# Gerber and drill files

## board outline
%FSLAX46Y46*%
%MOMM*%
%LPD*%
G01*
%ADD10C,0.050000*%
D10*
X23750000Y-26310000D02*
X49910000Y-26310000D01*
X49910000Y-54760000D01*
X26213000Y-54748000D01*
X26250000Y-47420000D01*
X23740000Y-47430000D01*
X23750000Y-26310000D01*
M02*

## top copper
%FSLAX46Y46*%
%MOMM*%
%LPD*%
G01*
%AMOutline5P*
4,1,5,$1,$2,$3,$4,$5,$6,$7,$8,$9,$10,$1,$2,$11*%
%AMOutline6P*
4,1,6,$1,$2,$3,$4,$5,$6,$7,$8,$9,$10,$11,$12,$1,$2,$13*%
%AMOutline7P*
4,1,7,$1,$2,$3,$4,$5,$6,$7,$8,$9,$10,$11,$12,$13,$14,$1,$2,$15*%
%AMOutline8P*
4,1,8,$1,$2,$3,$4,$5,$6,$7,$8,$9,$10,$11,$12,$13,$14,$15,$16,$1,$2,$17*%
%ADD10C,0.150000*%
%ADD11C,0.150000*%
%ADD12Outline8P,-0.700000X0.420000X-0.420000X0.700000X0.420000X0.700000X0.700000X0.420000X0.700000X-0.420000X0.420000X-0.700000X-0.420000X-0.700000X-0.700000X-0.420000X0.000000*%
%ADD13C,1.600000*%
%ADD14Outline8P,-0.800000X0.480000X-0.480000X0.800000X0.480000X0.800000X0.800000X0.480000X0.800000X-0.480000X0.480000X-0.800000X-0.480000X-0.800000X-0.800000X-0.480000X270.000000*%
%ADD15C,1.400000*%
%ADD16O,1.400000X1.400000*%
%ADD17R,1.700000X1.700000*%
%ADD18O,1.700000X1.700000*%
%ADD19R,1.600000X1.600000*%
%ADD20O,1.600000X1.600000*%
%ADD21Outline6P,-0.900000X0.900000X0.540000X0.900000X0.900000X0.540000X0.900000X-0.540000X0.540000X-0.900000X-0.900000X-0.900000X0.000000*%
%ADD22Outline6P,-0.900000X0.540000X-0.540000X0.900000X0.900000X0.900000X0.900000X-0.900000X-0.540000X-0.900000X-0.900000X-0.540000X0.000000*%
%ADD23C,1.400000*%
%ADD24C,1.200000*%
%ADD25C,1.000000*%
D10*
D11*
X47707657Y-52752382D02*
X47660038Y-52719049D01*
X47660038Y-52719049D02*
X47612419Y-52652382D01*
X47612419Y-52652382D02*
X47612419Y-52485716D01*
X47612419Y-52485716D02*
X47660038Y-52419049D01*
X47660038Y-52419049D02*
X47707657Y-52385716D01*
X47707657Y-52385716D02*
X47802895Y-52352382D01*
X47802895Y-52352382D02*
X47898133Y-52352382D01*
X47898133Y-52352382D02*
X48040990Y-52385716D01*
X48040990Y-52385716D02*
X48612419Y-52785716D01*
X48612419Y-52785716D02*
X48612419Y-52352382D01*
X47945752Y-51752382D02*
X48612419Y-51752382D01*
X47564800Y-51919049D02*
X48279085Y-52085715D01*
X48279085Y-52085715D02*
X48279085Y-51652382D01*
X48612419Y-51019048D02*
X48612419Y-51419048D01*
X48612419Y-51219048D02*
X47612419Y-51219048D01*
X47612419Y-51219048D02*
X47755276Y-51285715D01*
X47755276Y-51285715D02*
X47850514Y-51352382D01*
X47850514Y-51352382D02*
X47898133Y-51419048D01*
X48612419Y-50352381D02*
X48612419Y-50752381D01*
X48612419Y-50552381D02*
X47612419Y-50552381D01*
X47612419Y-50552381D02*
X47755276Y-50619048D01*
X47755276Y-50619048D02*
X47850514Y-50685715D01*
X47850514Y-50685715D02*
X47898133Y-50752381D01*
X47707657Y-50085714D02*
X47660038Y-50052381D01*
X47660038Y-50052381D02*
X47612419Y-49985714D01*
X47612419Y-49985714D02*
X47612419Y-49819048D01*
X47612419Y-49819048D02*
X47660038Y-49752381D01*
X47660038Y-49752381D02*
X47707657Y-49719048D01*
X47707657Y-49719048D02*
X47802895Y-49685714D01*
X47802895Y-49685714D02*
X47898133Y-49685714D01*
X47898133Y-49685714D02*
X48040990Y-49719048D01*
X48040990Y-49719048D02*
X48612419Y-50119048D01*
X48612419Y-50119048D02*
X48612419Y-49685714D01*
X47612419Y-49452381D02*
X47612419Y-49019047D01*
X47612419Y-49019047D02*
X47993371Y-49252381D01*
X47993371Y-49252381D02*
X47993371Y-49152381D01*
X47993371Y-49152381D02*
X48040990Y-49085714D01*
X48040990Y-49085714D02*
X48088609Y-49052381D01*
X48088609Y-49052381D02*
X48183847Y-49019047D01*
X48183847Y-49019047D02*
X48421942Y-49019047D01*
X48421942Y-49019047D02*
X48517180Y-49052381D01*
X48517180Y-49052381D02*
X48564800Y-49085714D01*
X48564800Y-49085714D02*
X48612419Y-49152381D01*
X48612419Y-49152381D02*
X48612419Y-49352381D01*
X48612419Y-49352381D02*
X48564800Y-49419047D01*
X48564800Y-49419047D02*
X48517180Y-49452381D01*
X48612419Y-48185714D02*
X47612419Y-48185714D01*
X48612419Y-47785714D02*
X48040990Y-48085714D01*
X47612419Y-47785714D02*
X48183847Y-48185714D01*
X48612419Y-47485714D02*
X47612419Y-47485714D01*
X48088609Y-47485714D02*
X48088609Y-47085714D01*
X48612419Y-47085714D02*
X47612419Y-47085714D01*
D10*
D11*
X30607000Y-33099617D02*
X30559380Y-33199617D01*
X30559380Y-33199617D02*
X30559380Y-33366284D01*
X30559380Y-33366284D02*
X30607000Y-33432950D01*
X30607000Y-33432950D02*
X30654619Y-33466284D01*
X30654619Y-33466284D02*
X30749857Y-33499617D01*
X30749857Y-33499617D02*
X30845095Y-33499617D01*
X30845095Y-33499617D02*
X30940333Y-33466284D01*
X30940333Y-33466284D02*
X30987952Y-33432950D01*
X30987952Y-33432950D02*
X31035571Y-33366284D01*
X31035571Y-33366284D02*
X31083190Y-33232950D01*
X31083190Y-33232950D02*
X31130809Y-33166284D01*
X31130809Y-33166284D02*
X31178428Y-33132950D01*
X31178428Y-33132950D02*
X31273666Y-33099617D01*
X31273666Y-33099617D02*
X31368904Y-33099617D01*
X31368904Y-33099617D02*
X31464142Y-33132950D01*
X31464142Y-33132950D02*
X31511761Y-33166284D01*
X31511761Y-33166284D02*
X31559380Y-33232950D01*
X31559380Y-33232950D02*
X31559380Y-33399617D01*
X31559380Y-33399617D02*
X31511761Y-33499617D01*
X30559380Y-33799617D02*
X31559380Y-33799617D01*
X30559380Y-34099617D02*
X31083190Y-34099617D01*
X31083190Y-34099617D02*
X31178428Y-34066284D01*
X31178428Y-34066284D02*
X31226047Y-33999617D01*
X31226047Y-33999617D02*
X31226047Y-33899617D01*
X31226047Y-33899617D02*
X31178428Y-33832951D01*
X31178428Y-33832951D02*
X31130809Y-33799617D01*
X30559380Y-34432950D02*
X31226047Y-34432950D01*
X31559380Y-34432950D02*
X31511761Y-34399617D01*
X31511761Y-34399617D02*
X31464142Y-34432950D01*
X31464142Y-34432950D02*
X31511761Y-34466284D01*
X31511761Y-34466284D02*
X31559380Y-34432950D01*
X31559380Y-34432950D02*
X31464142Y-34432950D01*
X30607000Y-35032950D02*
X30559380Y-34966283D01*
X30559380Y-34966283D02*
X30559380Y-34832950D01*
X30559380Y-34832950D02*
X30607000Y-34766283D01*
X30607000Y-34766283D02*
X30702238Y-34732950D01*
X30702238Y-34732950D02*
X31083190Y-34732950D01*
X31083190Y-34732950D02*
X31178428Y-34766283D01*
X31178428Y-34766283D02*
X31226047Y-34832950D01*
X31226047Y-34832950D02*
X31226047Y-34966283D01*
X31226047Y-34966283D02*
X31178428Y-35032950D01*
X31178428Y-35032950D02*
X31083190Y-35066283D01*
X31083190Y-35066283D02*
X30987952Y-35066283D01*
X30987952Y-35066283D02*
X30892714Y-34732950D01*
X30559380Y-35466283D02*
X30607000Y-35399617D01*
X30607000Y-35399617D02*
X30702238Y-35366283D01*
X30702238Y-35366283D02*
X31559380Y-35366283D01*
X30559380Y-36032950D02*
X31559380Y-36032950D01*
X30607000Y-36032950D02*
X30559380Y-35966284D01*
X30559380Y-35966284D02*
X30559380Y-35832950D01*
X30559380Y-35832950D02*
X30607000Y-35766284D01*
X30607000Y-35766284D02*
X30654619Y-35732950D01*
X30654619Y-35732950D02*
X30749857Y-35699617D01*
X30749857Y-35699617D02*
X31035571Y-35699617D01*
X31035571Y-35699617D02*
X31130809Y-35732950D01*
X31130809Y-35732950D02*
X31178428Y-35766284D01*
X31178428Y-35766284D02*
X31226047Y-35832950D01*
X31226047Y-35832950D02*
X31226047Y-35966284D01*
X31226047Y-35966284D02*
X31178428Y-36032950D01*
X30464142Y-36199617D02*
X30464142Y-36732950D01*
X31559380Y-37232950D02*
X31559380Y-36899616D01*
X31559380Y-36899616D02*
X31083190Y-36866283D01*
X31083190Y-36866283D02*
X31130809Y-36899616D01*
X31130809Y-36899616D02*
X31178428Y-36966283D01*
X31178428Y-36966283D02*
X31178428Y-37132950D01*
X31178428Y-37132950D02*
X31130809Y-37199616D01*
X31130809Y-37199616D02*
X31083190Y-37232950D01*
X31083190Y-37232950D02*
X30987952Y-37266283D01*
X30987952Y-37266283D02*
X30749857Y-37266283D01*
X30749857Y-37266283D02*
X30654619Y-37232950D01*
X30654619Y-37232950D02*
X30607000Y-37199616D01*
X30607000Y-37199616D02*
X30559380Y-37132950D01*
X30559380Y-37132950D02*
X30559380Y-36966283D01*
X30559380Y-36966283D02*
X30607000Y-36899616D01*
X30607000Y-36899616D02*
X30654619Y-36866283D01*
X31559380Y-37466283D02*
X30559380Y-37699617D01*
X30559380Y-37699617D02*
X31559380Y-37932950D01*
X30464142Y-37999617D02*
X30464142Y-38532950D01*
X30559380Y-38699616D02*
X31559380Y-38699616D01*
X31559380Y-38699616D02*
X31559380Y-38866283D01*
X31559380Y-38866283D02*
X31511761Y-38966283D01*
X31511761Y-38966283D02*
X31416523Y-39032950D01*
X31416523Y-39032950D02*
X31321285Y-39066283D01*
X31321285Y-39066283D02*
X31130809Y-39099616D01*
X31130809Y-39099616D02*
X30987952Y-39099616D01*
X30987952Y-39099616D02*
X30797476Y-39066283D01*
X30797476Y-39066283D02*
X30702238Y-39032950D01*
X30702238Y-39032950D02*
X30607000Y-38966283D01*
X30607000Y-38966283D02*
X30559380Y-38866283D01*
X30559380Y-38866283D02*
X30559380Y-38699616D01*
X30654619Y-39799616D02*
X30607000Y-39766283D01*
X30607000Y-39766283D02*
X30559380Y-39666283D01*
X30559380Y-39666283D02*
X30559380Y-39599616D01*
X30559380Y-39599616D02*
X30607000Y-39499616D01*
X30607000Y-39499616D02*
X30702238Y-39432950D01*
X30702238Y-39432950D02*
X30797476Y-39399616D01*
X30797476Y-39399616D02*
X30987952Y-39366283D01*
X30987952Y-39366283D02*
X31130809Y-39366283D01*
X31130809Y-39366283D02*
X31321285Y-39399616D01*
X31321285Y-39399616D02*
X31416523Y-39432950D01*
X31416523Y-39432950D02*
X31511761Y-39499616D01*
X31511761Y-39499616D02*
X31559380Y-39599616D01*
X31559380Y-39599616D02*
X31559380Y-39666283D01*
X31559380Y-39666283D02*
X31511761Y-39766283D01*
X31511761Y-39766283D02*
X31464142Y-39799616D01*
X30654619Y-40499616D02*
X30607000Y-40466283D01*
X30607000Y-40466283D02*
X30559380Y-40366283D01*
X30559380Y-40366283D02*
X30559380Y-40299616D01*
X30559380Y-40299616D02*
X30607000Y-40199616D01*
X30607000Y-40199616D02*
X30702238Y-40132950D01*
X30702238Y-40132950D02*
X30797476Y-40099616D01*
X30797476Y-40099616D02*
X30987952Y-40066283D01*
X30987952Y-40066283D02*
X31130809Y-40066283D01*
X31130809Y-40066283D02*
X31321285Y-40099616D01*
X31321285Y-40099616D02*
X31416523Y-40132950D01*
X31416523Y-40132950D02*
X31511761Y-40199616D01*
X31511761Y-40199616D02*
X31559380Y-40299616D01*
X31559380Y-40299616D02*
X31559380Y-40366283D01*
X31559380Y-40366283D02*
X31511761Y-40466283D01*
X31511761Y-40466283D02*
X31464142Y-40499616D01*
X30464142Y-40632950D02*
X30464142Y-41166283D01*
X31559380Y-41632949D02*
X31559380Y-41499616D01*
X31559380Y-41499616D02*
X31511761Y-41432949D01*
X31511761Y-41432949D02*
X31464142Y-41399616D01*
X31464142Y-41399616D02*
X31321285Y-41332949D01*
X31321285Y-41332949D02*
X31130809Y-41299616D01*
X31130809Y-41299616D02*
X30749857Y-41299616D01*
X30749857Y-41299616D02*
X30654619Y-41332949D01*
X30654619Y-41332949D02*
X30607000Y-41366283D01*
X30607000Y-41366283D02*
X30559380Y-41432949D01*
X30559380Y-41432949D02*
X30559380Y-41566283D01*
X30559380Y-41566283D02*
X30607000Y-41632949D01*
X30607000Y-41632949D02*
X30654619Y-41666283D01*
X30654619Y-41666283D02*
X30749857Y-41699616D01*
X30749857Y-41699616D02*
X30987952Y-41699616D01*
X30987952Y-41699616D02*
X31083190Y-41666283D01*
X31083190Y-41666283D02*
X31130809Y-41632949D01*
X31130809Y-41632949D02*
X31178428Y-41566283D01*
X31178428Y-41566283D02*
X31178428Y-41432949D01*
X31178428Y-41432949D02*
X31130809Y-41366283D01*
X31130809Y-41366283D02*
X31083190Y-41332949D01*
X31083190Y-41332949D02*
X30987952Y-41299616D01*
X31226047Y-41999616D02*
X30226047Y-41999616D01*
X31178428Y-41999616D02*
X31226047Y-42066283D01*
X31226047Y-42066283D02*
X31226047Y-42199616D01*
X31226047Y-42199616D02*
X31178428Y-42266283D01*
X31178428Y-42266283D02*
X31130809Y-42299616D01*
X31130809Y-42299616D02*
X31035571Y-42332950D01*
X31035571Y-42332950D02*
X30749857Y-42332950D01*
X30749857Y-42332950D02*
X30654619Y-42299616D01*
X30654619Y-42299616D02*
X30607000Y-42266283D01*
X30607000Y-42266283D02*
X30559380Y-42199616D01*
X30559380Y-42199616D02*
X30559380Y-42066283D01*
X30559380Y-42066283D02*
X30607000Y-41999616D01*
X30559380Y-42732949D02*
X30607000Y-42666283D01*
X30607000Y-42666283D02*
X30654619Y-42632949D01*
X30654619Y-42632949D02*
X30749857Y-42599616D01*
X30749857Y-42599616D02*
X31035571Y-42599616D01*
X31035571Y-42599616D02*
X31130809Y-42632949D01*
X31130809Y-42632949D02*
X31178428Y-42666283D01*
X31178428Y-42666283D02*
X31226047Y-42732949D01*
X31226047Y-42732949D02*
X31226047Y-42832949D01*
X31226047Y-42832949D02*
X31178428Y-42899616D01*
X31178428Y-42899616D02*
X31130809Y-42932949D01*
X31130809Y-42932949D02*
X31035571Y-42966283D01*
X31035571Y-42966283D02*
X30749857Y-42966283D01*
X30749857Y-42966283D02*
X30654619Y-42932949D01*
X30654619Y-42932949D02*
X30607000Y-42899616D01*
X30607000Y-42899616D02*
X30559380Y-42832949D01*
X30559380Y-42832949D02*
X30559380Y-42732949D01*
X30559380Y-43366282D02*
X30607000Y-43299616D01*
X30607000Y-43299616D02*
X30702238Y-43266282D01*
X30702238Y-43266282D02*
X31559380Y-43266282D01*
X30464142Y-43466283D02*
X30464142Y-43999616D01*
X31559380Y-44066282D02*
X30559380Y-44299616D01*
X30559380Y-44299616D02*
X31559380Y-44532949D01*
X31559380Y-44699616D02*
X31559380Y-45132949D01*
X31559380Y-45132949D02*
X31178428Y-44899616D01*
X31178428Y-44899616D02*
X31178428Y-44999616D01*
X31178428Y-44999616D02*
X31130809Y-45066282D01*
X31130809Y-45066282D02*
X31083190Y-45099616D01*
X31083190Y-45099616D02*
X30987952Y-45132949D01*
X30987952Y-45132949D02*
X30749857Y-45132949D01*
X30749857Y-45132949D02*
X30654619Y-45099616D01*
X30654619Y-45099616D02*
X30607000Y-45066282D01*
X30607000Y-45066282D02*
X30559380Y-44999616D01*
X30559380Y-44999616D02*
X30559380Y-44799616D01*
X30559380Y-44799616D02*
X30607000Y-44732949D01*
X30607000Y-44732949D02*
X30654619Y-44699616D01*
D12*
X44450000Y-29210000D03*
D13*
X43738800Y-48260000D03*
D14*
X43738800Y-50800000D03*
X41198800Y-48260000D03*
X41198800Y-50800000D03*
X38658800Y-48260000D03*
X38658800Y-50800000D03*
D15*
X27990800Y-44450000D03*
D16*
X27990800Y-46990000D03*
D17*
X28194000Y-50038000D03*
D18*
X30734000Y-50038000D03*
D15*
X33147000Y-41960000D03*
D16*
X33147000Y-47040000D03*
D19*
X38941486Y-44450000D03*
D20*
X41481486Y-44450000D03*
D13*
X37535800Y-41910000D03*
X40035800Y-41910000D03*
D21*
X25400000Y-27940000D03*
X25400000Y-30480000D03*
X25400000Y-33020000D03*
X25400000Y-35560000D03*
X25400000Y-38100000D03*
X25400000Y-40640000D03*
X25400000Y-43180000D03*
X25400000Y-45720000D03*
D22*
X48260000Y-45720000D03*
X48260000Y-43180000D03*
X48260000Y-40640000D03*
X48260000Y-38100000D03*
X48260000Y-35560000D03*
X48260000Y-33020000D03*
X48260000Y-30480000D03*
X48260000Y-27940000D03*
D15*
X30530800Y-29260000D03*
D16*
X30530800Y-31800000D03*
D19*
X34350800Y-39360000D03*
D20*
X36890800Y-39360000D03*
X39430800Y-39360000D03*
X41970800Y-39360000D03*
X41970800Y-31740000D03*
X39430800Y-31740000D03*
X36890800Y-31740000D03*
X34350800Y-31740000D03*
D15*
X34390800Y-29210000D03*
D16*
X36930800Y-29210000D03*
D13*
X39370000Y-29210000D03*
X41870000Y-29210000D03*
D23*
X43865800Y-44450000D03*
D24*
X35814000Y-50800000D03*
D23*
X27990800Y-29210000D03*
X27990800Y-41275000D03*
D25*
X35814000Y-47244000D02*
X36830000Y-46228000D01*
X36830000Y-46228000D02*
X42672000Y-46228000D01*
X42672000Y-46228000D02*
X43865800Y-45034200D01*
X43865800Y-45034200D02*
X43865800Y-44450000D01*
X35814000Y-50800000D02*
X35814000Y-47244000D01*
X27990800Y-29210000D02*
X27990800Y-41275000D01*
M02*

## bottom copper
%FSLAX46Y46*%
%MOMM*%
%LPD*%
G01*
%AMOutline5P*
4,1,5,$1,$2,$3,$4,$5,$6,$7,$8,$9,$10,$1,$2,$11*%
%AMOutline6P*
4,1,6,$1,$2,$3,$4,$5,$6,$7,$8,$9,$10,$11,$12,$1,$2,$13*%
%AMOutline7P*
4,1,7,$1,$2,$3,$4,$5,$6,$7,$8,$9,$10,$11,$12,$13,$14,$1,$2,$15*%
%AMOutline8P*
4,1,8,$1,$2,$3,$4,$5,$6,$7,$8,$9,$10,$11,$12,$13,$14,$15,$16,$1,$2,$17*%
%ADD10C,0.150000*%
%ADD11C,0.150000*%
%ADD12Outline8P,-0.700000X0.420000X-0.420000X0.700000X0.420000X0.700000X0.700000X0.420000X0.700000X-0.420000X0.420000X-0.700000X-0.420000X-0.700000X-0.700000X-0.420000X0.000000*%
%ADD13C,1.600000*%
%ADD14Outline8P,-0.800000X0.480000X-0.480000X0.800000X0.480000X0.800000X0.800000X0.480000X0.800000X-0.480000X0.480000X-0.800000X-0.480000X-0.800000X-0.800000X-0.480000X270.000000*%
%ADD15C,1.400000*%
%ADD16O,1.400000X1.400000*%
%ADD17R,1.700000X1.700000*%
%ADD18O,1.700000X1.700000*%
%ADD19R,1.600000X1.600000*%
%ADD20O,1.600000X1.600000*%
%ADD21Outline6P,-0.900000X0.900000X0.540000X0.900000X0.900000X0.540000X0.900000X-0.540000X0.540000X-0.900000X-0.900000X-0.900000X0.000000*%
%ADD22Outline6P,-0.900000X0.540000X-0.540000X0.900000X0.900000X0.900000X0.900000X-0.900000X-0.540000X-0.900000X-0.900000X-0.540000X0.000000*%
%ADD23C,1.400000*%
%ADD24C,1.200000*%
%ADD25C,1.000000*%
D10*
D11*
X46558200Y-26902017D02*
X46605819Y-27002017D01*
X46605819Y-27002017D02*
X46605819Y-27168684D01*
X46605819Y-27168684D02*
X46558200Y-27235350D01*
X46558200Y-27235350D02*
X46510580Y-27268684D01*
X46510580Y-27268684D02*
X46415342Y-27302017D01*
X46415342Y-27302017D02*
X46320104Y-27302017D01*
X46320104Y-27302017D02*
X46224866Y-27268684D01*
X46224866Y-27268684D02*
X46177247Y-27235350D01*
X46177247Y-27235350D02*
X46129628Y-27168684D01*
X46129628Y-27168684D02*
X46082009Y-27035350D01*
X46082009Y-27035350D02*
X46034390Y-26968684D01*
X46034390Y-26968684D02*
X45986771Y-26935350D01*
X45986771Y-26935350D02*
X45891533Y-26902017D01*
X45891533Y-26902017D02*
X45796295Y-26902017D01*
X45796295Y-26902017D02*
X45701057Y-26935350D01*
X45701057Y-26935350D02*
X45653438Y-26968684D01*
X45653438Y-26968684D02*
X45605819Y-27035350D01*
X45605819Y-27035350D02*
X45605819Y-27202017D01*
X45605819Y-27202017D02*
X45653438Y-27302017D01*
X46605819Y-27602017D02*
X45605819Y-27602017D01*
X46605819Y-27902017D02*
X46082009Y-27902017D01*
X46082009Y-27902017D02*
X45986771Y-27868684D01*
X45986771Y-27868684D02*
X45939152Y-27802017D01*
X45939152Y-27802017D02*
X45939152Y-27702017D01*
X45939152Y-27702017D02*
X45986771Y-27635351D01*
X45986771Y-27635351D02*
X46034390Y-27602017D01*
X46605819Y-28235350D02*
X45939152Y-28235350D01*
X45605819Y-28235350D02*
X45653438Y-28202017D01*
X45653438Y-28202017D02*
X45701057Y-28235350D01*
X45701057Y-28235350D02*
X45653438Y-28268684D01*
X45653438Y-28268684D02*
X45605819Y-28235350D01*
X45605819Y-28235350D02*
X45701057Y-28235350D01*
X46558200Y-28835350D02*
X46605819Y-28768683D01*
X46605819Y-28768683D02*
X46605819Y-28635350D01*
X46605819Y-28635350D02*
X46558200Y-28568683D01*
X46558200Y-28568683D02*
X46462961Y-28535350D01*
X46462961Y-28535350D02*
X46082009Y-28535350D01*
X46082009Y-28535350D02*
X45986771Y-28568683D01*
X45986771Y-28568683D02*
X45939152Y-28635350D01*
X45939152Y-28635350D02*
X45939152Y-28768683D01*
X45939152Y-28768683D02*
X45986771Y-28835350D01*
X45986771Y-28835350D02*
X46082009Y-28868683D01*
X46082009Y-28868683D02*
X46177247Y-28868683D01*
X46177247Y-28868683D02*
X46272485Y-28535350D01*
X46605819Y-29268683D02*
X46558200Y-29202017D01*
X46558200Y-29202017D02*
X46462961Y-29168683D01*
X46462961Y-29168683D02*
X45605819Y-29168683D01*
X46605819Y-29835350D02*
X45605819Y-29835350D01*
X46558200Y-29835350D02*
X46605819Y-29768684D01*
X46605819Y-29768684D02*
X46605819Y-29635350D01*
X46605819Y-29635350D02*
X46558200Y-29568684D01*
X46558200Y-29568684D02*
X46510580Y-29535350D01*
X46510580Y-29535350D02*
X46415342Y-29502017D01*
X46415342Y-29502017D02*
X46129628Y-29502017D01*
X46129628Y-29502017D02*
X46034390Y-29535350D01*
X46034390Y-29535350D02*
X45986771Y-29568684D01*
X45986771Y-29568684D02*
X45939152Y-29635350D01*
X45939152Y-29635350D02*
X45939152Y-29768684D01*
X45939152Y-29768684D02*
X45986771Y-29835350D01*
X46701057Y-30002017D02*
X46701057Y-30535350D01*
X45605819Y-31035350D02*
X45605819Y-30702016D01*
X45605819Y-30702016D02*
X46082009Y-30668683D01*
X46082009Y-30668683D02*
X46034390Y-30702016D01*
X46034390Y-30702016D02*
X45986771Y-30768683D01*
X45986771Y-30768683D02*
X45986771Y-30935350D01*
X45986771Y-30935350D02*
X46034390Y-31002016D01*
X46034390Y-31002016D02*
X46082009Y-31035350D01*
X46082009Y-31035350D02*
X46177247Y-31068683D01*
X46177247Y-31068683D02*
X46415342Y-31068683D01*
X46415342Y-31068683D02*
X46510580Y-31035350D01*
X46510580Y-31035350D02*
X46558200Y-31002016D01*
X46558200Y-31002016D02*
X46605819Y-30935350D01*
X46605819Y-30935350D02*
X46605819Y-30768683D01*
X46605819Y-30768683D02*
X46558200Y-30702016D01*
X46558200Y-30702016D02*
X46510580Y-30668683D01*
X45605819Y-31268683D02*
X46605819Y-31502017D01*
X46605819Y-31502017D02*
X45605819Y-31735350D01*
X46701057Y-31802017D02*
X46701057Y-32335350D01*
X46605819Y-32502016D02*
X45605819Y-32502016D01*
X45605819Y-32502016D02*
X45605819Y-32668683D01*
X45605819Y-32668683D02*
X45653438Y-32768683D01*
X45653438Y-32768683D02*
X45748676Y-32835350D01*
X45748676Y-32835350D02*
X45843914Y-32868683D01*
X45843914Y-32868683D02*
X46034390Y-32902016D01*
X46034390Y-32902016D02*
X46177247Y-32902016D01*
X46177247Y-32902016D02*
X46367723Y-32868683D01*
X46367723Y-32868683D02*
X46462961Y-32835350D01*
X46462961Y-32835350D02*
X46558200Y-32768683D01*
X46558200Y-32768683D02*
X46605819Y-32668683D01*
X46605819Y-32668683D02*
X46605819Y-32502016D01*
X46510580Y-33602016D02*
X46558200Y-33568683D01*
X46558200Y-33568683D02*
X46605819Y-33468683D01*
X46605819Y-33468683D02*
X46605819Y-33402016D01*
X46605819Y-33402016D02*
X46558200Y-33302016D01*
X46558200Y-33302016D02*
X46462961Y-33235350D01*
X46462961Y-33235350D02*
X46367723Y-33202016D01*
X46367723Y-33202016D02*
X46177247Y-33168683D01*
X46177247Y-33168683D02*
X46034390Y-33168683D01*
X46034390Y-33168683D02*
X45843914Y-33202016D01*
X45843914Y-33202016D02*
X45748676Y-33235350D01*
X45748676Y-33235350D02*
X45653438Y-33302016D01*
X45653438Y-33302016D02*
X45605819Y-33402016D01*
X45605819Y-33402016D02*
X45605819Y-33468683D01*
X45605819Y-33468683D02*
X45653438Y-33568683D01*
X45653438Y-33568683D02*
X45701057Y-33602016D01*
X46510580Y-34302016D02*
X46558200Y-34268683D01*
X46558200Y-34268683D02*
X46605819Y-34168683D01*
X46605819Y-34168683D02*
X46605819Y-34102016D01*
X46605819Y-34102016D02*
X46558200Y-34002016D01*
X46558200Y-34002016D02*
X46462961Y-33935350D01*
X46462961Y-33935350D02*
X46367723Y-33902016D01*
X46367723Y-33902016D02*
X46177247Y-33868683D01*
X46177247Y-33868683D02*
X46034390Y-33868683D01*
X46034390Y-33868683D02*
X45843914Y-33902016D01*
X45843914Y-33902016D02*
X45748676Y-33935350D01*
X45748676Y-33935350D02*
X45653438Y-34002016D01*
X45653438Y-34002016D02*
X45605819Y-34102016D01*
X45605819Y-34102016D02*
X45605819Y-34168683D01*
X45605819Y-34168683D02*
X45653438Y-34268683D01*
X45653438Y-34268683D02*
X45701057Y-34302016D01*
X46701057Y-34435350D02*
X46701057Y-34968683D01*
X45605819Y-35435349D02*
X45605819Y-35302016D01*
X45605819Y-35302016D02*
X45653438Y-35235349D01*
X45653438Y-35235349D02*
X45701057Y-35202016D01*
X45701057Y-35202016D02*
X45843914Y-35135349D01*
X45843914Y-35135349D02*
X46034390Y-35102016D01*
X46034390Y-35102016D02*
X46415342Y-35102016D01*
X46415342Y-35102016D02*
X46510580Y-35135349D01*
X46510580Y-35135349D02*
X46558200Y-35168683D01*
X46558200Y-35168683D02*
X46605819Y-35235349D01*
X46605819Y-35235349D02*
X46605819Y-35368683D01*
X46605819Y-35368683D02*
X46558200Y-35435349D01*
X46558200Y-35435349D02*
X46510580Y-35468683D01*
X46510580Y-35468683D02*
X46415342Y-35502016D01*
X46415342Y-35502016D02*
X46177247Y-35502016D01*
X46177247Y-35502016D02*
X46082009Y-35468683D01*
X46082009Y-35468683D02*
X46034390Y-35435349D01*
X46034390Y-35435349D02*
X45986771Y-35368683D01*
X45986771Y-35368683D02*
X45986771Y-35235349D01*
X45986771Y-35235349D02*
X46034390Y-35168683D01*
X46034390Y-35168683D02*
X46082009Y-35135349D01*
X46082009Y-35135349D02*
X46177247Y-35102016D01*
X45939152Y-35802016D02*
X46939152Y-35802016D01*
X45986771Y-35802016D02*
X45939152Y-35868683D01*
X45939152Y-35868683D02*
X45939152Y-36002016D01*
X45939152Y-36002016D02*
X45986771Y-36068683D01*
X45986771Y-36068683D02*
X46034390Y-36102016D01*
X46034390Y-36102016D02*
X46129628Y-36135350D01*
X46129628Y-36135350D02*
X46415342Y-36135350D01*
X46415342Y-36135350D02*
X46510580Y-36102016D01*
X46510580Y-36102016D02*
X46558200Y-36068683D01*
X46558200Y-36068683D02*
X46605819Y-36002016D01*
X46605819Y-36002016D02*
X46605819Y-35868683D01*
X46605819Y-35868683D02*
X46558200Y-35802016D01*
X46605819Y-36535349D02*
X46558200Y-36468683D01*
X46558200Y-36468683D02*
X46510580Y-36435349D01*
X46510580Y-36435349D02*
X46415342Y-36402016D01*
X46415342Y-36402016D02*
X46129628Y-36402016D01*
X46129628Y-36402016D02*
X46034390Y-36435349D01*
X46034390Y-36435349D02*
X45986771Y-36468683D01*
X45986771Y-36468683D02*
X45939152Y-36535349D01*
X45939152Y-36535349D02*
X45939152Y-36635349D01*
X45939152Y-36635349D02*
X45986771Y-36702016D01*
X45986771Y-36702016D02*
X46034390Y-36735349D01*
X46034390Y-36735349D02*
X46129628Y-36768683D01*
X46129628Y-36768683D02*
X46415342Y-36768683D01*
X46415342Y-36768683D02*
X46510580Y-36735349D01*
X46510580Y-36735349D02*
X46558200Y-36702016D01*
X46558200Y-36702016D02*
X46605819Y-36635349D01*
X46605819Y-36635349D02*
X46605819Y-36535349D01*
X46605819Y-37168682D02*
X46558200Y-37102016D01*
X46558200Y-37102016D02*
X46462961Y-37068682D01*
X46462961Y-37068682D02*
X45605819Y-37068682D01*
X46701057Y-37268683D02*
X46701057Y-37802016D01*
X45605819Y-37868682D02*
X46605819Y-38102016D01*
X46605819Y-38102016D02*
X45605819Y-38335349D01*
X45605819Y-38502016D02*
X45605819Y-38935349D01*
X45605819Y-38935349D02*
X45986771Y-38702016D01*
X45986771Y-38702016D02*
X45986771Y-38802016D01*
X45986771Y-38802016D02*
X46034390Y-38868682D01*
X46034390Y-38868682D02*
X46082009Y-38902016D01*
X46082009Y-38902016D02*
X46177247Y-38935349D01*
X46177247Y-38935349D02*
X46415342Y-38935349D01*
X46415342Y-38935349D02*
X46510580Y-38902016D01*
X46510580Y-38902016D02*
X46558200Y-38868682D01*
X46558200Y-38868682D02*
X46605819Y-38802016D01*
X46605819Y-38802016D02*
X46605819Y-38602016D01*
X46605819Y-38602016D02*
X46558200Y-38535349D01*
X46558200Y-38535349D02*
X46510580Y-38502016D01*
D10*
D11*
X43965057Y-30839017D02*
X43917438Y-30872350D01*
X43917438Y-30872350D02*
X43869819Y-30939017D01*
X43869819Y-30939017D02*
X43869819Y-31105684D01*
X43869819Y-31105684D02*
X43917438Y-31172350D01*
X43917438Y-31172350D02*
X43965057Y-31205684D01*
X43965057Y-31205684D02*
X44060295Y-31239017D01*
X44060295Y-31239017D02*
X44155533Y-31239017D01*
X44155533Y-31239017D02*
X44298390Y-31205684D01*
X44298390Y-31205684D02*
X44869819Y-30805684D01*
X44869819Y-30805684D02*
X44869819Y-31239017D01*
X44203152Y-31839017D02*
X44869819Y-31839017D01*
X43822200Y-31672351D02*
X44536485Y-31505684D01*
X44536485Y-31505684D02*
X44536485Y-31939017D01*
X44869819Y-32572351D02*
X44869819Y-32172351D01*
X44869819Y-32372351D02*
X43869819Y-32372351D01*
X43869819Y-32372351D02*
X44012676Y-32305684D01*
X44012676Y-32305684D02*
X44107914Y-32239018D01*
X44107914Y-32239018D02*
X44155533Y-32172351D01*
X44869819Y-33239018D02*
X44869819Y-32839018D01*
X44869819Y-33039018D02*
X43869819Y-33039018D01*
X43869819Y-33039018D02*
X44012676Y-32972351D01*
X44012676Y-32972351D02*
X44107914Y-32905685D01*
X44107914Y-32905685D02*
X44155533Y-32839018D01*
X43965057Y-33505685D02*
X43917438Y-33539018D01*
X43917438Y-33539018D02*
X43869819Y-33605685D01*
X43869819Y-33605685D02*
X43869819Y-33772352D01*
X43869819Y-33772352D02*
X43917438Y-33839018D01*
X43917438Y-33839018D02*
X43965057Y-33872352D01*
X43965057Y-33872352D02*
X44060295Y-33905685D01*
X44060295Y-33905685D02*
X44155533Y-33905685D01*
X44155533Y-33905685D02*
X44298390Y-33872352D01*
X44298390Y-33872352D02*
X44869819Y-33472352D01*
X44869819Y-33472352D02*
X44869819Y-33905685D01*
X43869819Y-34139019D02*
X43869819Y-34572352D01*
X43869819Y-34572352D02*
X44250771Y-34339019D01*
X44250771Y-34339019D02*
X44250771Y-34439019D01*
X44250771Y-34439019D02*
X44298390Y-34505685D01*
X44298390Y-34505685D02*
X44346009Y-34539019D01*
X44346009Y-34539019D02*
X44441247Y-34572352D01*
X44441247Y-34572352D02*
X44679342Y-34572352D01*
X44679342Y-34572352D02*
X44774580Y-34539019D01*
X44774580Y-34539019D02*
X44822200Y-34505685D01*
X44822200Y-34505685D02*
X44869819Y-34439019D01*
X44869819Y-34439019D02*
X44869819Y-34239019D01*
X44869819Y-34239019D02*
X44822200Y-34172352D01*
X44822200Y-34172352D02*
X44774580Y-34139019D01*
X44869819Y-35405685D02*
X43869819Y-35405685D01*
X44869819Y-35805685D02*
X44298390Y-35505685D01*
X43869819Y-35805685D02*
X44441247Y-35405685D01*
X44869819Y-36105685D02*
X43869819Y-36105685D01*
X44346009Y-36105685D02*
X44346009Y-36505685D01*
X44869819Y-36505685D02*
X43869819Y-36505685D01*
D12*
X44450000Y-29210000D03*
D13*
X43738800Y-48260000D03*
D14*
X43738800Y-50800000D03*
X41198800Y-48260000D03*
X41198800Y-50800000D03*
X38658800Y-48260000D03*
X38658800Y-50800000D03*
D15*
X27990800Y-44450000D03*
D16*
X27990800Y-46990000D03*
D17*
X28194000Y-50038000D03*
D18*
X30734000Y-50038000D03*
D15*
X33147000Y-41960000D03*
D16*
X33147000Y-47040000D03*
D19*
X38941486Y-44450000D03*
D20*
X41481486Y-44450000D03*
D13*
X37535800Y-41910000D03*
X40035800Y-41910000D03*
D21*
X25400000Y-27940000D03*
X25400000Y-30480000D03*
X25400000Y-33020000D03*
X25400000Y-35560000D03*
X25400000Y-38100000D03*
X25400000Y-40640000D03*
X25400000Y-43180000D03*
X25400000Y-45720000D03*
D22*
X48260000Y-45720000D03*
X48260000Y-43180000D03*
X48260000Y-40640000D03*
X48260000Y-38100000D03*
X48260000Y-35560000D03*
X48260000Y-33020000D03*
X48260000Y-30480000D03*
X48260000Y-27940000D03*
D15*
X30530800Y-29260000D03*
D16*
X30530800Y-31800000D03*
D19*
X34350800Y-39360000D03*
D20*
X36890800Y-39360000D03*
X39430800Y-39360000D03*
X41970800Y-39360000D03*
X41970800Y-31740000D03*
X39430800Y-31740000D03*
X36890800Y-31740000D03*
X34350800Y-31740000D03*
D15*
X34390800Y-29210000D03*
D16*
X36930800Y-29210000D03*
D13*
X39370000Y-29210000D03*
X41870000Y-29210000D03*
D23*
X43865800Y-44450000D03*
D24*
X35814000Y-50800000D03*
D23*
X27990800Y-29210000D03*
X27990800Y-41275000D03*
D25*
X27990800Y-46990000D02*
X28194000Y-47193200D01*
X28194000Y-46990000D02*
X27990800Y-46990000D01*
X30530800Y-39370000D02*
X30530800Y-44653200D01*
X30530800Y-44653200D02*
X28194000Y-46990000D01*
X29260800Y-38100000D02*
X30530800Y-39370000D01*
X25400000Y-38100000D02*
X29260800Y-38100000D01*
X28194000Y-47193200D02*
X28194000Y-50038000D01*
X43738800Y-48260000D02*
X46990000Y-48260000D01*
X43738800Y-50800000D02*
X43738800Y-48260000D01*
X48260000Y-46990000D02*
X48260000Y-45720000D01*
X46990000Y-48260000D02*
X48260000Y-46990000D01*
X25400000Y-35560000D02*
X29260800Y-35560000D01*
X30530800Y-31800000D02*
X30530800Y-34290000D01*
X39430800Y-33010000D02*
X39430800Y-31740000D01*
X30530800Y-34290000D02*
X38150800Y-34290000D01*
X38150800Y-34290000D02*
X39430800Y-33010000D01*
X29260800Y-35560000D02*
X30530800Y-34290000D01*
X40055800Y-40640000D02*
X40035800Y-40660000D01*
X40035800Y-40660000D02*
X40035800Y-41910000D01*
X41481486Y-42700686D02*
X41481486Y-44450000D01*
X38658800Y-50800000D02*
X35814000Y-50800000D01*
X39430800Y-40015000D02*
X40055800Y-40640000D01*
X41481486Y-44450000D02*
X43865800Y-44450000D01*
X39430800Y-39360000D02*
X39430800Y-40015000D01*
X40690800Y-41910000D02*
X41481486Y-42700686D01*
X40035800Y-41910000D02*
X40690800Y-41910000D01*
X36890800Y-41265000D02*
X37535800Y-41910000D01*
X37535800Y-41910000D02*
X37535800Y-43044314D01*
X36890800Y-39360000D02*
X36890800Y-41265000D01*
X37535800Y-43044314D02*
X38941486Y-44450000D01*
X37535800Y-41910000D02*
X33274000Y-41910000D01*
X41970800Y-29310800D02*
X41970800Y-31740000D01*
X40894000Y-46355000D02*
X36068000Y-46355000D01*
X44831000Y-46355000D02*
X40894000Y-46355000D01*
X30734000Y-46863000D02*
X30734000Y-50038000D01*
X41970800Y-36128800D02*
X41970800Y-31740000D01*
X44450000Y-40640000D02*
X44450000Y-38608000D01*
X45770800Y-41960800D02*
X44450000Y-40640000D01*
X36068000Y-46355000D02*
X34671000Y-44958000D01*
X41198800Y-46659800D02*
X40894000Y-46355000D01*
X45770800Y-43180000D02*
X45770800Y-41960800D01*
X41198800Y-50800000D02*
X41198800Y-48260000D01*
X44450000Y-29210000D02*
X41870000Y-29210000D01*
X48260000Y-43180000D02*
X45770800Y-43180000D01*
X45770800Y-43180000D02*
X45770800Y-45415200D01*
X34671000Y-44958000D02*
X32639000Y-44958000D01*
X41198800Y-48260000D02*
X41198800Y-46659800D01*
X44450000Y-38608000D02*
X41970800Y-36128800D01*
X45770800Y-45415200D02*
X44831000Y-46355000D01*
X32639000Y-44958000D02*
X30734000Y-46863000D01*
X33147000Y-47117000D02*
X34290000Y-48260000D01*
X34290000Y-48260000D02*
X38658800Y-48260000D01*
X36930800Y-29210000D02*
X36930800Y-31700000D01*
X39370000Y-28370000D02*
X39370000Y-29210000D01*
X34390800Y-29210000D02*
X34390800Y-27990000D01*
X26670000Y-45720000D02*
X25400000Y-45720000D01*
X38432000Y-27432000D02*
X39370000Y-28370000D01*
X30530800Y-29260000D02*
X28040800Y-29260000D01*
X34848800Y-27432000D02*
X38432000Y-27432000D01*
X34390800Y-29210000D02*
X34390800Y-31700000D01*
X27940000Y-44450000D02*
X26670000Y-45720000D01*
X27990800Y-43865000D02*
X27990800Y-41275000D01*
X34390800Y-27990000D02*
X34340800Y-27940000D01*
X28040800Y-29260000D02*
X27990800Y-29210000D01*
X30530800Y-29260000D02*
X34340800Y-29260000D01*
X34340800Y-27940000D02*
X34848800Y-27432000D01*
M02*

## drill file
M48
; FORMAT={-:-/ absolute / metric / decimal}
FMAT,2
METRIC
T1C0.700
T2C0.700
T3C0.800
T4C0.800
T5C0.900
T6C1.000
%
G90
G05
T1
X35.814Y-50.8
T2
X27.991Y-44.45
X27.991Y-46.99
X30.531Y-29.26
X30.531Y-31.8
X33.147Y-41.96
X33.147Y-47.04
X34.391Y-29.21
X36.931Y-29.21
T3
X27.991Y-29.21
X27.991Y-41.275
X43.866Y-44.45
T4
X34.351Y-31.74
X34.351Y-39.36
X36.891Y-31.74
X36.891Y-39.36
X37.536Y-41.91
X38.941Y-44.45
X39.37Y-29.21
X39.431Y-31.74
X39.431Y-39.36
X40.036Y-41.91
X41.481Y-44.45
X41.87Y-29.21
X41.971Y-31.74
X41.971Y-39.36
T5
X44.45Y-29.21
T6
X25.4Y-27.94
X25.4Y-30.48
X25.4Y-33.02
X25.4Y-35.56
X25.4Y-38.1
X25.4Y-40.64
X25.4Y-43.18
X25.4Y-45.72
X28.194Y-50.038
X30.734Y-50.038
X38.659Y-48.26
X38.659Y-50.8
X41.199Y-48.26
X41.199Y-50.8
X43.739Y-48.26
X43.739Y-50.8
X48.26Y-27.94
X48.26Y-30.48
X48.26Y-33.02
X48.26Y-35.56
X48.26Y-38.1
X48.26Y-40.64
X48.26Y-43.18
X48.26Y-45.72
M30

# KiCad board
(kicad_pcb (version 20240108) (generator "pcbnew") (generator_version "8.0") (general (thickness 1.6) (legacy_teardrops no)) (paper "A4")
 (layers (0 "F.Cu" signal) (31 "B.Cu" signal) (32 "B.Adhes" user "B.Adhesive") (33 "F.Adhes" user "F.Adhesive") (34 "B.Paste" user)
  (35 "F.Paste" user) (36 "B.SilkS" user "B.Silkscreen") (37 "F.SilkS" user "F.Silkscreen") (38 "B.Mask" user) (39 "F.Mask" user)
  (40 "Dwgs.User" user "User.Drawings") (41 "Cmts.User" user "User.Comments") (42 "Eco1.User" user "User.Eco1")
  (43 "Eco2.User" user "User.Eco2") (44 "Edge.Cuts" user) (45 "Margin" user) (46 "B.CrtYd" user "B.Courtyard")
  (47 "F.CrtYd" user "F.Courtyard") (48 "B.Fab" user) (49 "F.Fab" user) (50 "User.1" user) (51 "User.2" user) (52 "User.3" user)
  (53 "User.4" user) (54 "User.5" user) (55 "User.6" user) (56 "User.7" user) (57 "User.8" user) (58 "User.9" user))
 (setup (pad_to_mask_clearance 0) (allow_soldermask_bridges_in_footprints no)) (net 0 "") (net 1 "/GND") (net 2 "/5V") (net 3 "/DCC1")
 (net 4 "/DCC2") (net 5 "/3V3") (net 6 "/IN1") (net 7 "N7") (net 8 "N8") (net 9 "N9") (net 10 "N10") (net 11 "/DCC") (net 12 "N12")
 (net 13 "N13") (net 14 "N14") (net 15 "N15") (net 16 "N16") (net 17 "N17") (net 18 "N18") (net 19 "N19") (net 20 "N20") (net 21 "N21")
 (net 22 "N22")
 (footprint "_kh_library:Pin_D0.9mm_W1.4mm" (layer "F.Cu") (at 44.45 29.21)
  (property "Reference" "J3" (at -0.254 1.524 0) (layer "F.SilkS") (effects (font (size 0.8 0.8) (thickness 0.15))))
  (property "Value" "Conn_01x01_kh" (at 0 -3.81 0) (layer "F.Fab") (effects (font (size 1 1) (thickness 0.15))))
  (pad "1" thru_hole roundrect (at 0 0) (size 1.4 1.4) (drill 0.9) (layers "*.Cu" "*.Mask") (remove_unused_layers no) (roundrect_rratio 0)
   (chamfer_ratio 0.2) (chamfer top_left top_right bottom_left bottom_right) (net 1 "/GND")))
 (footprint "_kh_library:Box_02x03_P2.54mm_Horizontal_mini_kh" (layer "F.Cu") (at 43.7388 48.26 -90)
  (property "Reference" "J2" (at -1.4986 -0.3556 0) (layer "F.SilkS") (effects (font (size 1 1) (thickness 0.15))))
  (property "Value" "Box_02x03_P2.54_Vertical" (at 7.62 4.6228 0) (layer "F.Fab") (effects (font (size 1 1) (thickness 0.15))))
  (pad "1" thru_hole circle (at 0 0 270) (size 1.6 1.6) (drill 1) (layers "*.Cu" "*.Mask") (remove_unused_layers no) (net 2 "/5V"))
  (pad "2" thru_hole roundrect (at 2.54 0 270) (size 1.6 1.6) (drill 1) (layers "*.Cu" "*.Mask") (remove_unused_layers no)
   (roundrect_rratio 0) (chamfer_ratio 0.2) (chamfer top_left top_right bottom_left bottom_right) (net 2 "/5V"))
  (pad "3" thru_hole roundrect (at 0 2.54 270) (size 1.6 1.6) (drill 1) (layers "*.Cu" "*.Mask") (remove_unused_layers no)
   (roundrect_rratio 0) (chamfer_ratio 0.2) (chamfer top_left top_right bottom_left bottom_right) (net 1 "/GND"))
  (pad "4" thru_hole roundrect (at 2.54 2.54 270) (size 1.6 1.6) (drill 1) (layers "*.Cu" "*.Mask") (remove_unused_layers no)
   (roundrect_rratio 0) (chamfer_ratio 0.2) (chamfer top_left top_right bottom_left bottom_right) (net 1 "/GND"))
  (pad "5" thru_hole roundrect (at 0 5.08 270) (size 1.6 1.6) (drill 1) (layers "*.Cu" "*.Mask") (remove_unused_layers no)
   (roundrect_rratio 0) (chamfer_ratio 0.2) (chamfer top_left top_right bottom_left bottom_right) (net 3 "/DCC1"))
  (pad "6" thru_hole roundrect (at 2.54 5.08 270) (size 1.6 1.6) (drill 1) (layers "*.Cu" "*.Mask") (remove_unused_layers no)
   (roundrect_rratio 0) (chamfer_ratio 0.2) (chamfer top_left top_right bottom_left bottom_right) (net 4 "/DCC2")))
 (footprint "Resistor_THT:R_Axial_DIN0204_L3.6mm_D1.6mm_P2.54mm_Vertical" (layer "F.Cu") (at 27.9908 44.45 -90)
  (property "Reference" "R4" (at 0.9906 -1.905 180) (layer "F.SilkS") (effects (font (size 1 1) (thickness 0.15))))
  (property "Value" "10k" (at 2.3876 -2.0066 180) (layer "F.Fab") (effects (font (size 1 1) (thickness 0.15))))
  (pad "1" thru_hole circle (at 0 0 270) (size 1.4 1.4) (drill 0.7) (layers "*.Cu" "*.Mask") (remove_unused_layers no) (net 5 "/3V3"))
  (pad "2" thru_hole oval (at 2.54 0 270) (size 1.4 1.4) (drill 0.7) (layers "*.Cu" "*.Mask") (remove_unused_layers no) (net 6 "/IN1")))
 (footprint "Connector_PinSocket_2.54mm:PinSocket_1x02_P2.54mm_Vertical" (layer "F.Cu") (at 28.194 50.038 90)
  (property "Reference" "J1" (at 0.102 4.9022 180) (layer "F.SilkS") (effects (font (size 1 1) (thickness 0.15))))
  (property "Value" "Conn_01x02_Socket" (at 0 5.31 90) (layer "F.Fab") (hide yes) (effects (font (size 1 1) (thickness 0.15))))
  (pad "1" thru_hole rect (at 0 0 90) (size 1.7 1.7) (drill 1) (layers "*.Cu" "*.Mask") (remove_unused_layers no) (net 6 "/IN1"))
  (pad "2" thru_hole oval (at 0 2.54 90) (size 1.7 1.7) (drill 1) (layers "*.Cu" "*.Mask") (remove_unused_layers no) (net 1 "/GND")))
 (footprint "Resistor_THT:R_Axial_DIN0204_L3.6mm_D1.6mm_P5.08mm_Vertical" (layer "F.Cu") (at 33.147 41.96 -90)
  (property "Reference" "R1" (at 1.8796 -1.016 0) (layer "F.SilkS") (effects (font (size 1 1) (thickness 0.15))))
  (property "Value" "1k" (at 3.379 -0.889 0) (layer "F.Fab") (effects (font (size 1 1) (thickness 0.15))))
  (pad "1" thru_hole circle (at 0 0 270) (size 1.4 1.4) (drill 0.7) (layers "*.Cu" "*.Mask") (remove_unused_layers no) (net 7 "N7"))
  (pad "2" thru_hole oval (at 5.08 0 270) (size 1.4 1.4) (drill 0.7) (layers "*.Cu" "*.Mask") (remove_unused_layers no) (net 3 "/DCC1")))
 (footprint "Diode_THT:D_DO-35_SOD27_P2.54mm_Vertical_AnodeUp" (layer "F.Cu") (at 38.941486 44.45)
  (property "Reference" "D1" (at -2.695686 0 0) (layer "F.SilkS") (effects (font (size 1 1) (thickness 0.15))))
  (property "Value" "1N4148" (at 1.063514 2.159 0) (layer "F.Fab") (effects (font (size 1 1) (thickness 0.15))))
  (pad "1" thru_hole rect (at 0 0) (size 1.6 1.6) (drill 0.8) (layers "*.Cu" "*.Mask") (remove_unused_layers no) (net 7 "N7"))
  (pad "2" thru_hole oval (at 2.54 0) (size 1.6 1.6) (drill 0.8) (layers "*.Cu" "*.Mask") (remove_unused_layers no) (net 4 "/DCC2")))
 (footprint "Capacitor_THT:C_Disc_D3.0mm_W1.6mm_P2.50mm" (layer "F.Cu") (at 37.5358 41.91)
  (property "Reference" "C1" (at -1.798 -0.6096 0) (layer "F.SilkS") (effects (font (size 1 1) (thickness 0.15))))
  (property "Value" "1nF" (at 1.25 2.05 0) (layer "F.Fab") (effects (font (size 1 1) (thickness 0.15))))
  (pad "1" thru_hole circle (at 0 0) (size 1.6 1.6) (drill 0.8) (layers "*.Cu" "*.Mask") (remove_unused_layers no) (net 7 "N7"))
  (pad "2" thru_hole circle (at 2.5 0) (size 1.6 1.6) (drill 0.8) (layers "*.Cu" "*.Mask") (remove_unused_layers no) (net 4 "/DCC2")))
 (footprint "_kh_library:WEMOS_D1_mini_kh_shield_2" (layer "F.Cu") (at 25.4 27.94)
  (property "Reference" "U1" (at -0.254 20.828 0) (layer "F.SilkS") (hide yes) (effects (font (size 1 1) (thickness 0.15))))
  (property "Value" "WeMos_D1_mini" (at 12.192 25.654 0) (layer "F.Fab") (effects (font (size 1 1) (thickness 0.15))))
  (pad "1" thru_hole roundrect (at 0 0) (size 1.8 1.8) (drill 1) (layers "*.Cu" "*.Mask") (remove_unused_layers no) (roundrect_rratio 0)
   (chamfer_ratio 0.2) (chamfer top_right bottom_right) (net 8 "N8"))
  (pad "2" thru_hole roundrect (at 0 2.54) (size 1.8 1.8) (drill 1) (layers "*.Cu" "*.Mask") (remove_unused_layers no) (roundrect_rratio 0)
   (chamfer_ratio 0.2) (chamfer top_right bottom_right) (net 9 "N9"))
  (pad "3" thru_hole roundrect (at 0 5.08) (size 1.8 1.8) (drill 1) (layers "*.Cu" "*.Mask") (remove_unused_layers no) (roundrect_rratio 0)
   (chamfer_ratio 0.2) (chamfer top_right bottom_right) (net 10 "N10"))
  (pad "4" thru_hole roundrect (at 0 7.62) (size 1.8 1.8) (drill 1) (layers "*.Cu" "*.Mask") (remove_unused_layers no) (roundrect_rratio 0)
   (chamfer_ratio 0.2) (chamfer top_right bottom_right) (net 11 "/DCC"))
  (pad "5" thru_hole roundrect (at 0 10.16) (size 1.8 1.8) (drill 1) (layers "*.Cu" "*.Mask") (remove_unused_layers no) (roundrect_rratio 0)
   (chamfer_ratio 0.2) (chamfer top_right bottom_right) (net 6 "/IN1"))
  (pad "6" thru_hole roundrect (at 0 12.7) (size 1.8 1.8) (drill 1) (layers "*.Cu" "*.Mask") (remove_unused_layers no) (roundrect_rratio 0)
   (chamfer_ratio 0.2) (chamfer top_right bottom_right) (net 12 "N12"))
  (pad "7" thru_hole roundrect (at 0 15.24) (size 1.8 1.8) (drill 1) (layers "*.Cu" "*.Mask") (remove_unused_layers no) (roundrect_rratio 0)
   (chamfer_ratio 0.2) (chamfer top_right bottom_right) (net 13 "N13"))
  (pad "8" thru_hole roundrect (at 0 17.78) (size 1.8 1.8) (drill 1) (layers "*.Cu" "*.Mask") (remove_unused_layers no) (roundrect_rratio 0)
   (chamfer_ratio 0.2) (chamfer top_right bottom_right) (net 5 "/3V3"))
  (pad "9" thru_hole roundrect (at 22.86 17.78) (size 1.8 1.8) (drill 1) (layers "*.Cu" "*.Mask") (remove_unused_layers no)
   (roundrect_rratio 0) (chamfer_ratio 0.2) (chamfer top_left bottom_left) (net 2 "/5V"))
  (pad "10" thru_hole roundrect (at 22.86 15.24) (size 1.8 1.8) (drill 1) (layers "*.Cu" "*.Mask") (remove_unused_layers no)
   (roundrect_rratio 0) (chamfer_ratio 0.2) (chamfer top_left bottom_left) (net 1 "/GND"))
  (pad "11" thru_hole roundrect (at 22.86 12.7) (size 1.8 1.8) (drill 1) (layers "*.Cu" "*.Mask") (remove_unused_layers no)
   (roundrect_rratio 0) (chamfer_ratio 0.2) (chamfer top_left bottom_left) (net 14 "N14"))
  (pad "12" thru_hole roundrect (at 22.86 10.16) (size 1.8 1.8) (drill 1) (layers "*.Cu" "*.Mask") (remove_unused_layers no)
   (roundrect_rratio 0) (chamfer_ratio 0.2) (chamfer top_left bottom_left) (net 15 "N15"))
  (pad "13" thru_hole roundrect (at 22.86 7.62) (size 1.8 1.8) (drill 1) (layers "*.Cu" "*.Mask") (remove_unused_layers no)
   (roundrect_rratio 0) (chamfer_ratio 0.2) (chamfer top_left bottom_left) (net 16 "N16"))
  (pad "14" thru_hole roundrect (at 22.86 5.08) (size 1.8 1.8) (drill 1) (layers "*.Cu" "*.Mask") (remove_unused_layers no)
   (roundrect_rratio 0) (chamfer_ratio 0.2) (chamfer top_left bottom_left) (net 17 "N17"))
  (pad "15" thru_hole roundrect (at 22.86 2.54) (size 1.8 1.8) (drill 1) (layers "*.Cu" "*.Mask") (remove_unused_layers no)
   (roundrect_rratio 0) (chamfer_ratio 0.2) (chamfer top_left bottom_left) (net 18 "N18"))
  (pad "16" thru_hole roundrect (at 22.86 0) (size 1.8 1.8) (drill 1) (layers "*.Cu" "*.Mask") (remove_unused_layers no)
   (roundrect_rratio 0) (chamfer_ratio 0.2) (chamfer top_left bottom_left) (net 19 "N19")))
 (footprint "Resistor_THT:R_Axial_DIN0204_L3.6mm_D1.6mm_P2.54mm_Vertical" (layer "F.Cu") (at 30.5308 29.26 -90)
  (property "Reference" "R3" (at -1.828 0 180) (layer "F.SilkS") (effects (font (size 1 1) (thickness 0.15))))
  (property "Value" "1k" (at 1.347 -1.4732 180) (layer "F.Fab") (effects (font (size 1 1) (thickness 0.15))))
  (pad "1" thru_hole circle (at 0 0 270) (size 1.4 1.4) (drill 0.7) (layers "*.Cu" "*.Mask") (remove_unused_layers no) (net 5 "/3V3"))
  (pad "2" thru_hole oval (at 2.54 0 270) (size 1.4 1.4) (drill 0.7) (layers "*.Cu" "*.Mask") (remove_unused_layers no) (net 11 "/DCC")))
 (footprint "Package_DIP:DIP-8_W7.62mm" (layer "F.Cu") (at 34.3508 39.36 90)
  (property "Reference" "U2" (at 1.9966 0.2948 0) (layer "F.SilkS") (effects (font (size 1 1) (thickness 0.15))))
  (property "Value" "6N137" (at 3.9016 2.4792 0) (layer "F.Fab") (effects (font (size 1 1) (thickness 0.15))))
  (pad "1" thru_hole rect (at 0 0 90) (size 1.6 1.6) (drill 0.8) (layers "*.Cu" "*.Mask") (remove_unused_layers no) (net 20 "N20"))
  (pad "2" thru_hole oval (at 0 2.54 90) (size 1.6 1.6) (drill 0.8) (layers "*.Cu" "*.Mask") (remove_unused_layers no) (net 7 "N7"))
  (pad "3" thru_hole oval (at 0 5.08 90) (size 1.6 1.6) (drill 0.8) (layers "*.Cu" "*.Mask") (remove_unused_layers no) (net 4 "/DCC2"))
  (pad "4" thru_hole oval (at 0 7.62 90) (size 1.6 1.6) (drill 0.8) (layers "*.Cu" "*.Mask") (remove_unused_layers no) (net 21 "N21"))
  (pad "5" thru_hole oval (at 7.62 7.62 90) (size 1.6 1.6) (drill 0.8) (layers "*.Cu" "*.Mask") (remove_unused_layers no) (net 1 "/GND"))
  (pad "6" thru_hole oval (at 7.62 5.08 90) (size 1.6 1.6) (drill 0.8) (layers "*.Cu" "*.Mask") (remove_unused_layers no) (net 11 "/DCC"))
  (pad "7" thru_hole oval (at 7.62 2.54 90) (size 1.6 1.6) (drill 0.8) (layers "*.Cu" "*.Mask") (remove_unused_layers no) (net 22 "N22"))
  (pad "8" thru_hole oval (at 7.62 0 90) (size 1.6 1.6) (drill 0.8) (layers "*.Cu" "*.Mask") (remove_unused_layers no) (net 5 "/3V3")))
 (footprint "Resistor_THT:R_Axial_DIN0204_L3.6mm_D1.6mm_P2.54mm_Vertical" (layer "F.Cu") (at 34.3908 29.21)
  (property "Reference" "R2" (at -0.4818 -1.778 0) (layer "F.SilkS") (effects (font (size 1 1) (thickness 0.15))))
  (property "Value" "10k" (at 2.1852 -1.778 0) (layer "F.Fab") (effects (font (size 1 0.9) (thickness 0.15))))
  (pad "1" thru_hole circle (at 0 0) (size 1.4 1.4) (drill 0.7) (layers "*.Cu" "*.Mask") (remove_unused_layers no) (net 5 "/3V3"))
  (pad "2" thru_hole oval (at 2.54 0) (size 1.4 1.4) (drill 0.7) (layers "*.Cu" "*.Mask") (remove_unused_layers no) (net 22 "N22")))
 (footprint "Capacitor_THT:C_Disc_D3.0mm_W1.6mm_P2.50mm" (layer "F.Cu") (at 39.37 29.21)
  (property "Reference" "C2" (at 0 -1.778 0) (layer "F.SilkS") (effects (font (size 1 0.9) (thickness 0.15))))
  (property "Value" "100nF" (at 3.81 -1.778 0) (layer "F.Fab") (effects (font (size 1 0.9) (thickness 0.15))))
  (pad "1" thru_hole circle (at 0 0) (size 1.6 1.6) (drill 0.8) (layers "*.Cu" "*.Mask") (remove_unused_layers no) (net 5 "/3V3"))
  (pad "2" thru_hole circle (at 2.5 0) (size 1.6 1.6) (drill 0.8) (layers "*.Cu" "*.Mask") (remove_unused_layers no) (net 1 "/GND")))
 (gr_poly
  (pts (xy 23.75 26.31) (xy 49.91 26.31) (xy 49.91 54.76) (xy 26.213 54.748) (xy 26.25 47.42) (xy 23.74 47.43))
  (stroke (width 0.05) (type solid)) (fill none) (layer "Edge.Cuts"))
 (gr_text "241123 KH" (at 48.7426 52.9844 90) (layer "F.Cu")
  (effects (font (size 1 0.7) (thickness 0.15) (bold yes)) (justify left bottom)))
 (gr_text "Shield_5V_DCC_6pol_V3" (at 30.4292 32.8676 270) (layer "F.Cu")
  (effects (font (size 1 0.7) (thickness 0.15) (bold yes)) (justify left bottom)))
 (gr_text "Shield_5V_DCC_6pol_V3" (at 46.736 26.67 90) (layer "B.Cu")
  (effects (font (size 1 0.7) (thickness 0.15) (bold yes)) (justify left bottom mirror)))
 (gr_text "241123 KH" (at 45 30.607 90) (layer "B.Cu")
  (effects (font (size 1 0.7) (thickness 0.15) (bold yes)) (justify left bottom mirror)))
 (segment (start 27.9908 46.99) (end 28.194 47.1932) (width 1) (layer "B.Cu") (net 6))
 (segment (start 28.194 46.99) (end 27.9908 46.99) (width 1) (layer "B.Cu") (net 6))
 (segment (start 30.5308 39.37) (end 30.5308 44.6532) (width 1) (layer "B.Cu") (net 6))
 (segment (start 30.5308 44.6532) (end 28.194 46.99) (width 1) (layer "B.Cu") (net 6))
 (segment (start 29.2608 38.1) (end 30.5308 39.37) (width 1) (layer "B.Cu") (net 6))
 (segment (start 25.4 38.1) (end 29.2608 38.1) (width 1) (layer "B.Cu") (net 6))
 (segment (start 28.194 47.1932) (end 28.194 50.038) (width 1) (layer "B.Cu") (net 6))
 (segment (start 43.7388 48.26) (end 46.99 48.26) (width 1) (layer "B.Cu") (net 2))
 (segment (start 43.7388 50.8) (end 43.7388 48.26) (width 1) (layer "B.Cu") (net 2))
 (segment (start 48.26 46.99) (end 48.26 45.72) (width 1) (layer "B.Cu") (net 2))
 (segment (start 46.99 48.26) (end 48.26 46.99) (width 1) (layer "B.Cu") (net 2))
 (segment (start 25.4 35.56) (end 29.2608 35.56) (width 1) (layer "B.Cu") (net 11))
 (segment (start 30.5308 31.8) (end 30.5308 34.29) (width 1) (layer "B.Cu") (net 11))
 (segment (start 39.4308 33.01) (end 39.4308 31.74) (width 1) (layer "B.Cu") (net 11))
 (segment (start 30.5308 34.29) (end 38.1508 34.29) (width 1) (layer "B.Cu") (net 11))
 (segment (start 38.1508 34.29) (end 39.4308 33.01) (width 1) (layer "B.Cu") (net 11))
 (segment (start 29.2608 35.56) (end 30.5308 34.29) (width 1) (layer "B.Cu") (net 11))
 (segment (start 35.814 47.244) (end 36.83 46.228) (width 1) (layer "F.Cu") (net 4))
 (segment (start 36.83 46.228) (end 42.672 46.228) (width 1) (layer "F.Cu") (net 4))
 (segment (start 42.672 46.228) (end 43.8658 45.0342) (width 1) (layer "F.Cu") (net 4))
 (segment (start 43.8658 45.0342) (end 43.8658 44.45) (width 1) (layer "F.Cu") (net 4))
 (segment (start 35.814 50.8) (end 35.814 47.244) (width 1) (layer "F.Cu") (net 4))
 (via (at 43.8658 44.45) (size 1.4) (drill 0.8) (layers "F.Cu" "B.Cu") (free yes) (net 4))
 (via (at 35.814 50.8) (size 1.2) (drill 0.7) (layers "F.Cu" "B.Cu") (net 4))
 (segment (start 40.0558 40.64) (end 40.0358 40.66) (width 1) (layer "B.Cu") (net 4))
 (segment (start 40.0358 40.66) (end 40.0358 41.91) (width 1) (layer "B.Cu") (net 4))
 (segment (start 41.481486 42.700686) (end 41.481486 44.45) (width 1) (layer "B.Cu") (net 4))
 (segment (start 38.6588 50.8) (end 35.814 50.8) (width 1) (layer "B.Cu") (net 4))
 (segment (start 39.4308 40.015) (end 40.0558 40.64) (width 1) (layer "B.Cu") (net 4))
 (segment (start 41.481486 44.45) (end 43.8658 44.45) (width 1) (layer "B.Cu") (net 4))
 (segment (start 39.4308 39.36) (end 39.4308 40.015) (width 1) (layer "B.Cu") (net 4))
 (segment (start 40.6908 41.91) (end 41.481486 42.700686) (width 1) (layer "B.Cu") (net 4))
 (segment (start 40.0358 41.91) (end 40.6908 41.91) (width 1) (layer "B.Cu") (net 4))
 (segment (start 36.8908 41.265) (end 37.5358 41.91) (width 1) (layer "B.Cu") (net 7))
 (segment (start 37.5358 41.91) (end 37.5358 43.044314) (width 1) (layer "B.Cu") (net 7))
 (segment (start 36.8908 39.36) (end 36.8908 41.265) (width 1) (layer "B.Cu") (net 7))
 (segment (start 37.5358 43.044314) (end 38.941486 44.45) (width 1) (layer "B.Cu") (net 7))
 (segment (start 37.5358 41.91) (end 33.274 41.91) (width 1) (layer "B.Cu") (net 7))
 (segment (start 41.9708 29.3108) (end 41.9708 31.74) (width 1) (layer "B.Cu") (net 1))
 (segment (start 40.894 46.355) (end 36.068 46.355) (width 1) (layer "B.Cu") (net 1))
 (segment (start 44.831 46.355) (end 40.894 46.355) (width 1) (layer "B.Cu") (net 1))
 (segment (start 30.734 46.863) (end 30.734 50.038) (width 1) (layer "B.Cu") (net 1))
 (segment (start 41.9708 36.1288) (end 41.9708 31.74) (width 1) (layer "B.Cu") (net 1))
 (segment (start 44.45 40.64) (end 44.45 38.608) (width 1) (layer "B.Cu") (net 1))
 (segment (start 45.7708 41.9608) (end 44.45 40.64) (width 1) (layer "B.Cu") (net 1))
 (segment (start 36.068 46.355) (end 34.671 44.958) (width 1) (layer "B.Cu") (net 1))
 (segment (start 41.1988 46.6598) (end 40.894 46.355) (width 1) (layer "B.Cu") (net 1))
 (segment (start 45.7708 43.18) (end 45.7708 41.9608) (width 1) (layer "B.Cu") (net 1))
 (segment (start 41.1988 50.8) (end 41.1988 48.26) (width 1) (layer "B.Cu") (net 1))
 (segment (start 44.45 29.21) (end 41.87 29.21) (width 1) (layer "B.Cu") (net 1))
 (segment (start 48.26 43.18) (end 45.7708 43.18) (width 1) (layer "B.Cu") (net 1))
 (segment (start 45.7708 43.18) (end 45.7708 45.4152) (width 1) (layer "B.Cu") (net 1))
 (segment (start 34.671 44.958) (end 32.639 44.958) (width 1) (layer "B.Cu") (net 1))
 (segment (start 41.1988 48.26) (end 41.1988 46.6598) (width 1) (layer "B.Cu") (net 1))
 (segment (start 44.45 38.608) (end 41.9708 36.1288) (width 1) (layer "B.Cu") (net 1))
 (segment (start 45.7708 45.4152) (end 44.831 46.355) (width 1) (layer "B.Cu") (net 1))
 (segment (start 32.639 44.958) (end 30.734 46.863) (width 1) (layer "B.Cu") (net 1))
 (segment (start 33.147 47.117) (end 34.29 48.26) (width 1) (layer "B.Cu") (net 3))
 (segment (start 34.29 48.26) (end 38.6588 48.26) (width 1) (layer "B.Cu") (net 3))
 (segment (start 36.9308 29.21) (end 36.9308 31.7) (width 1) (layer "B.Cu") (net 22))
 (segment (start 27.9908 29.21) (end 27.9908 41.275) (width 1) (layer "F.Cu") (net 5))
 (via (at 27.9908 29.21) (size 1.4) (drill 0.8) (layers "F.Cu" "B.Cu") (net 5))
 (via (at 27.9908 41.275) (size 1.4) (drill 0.8) (layers "F.Cu" "B.Cu") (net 5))
 (segment (start 39.37 28.37) (end 39.37 29.21) (width 1) (layer "B.Cu") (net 5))
 (segment (start 34.3908 29.21) (end 34.3908 27.99) (width 1) (layer "B.Cu") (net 5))
 (segment (start 26.67 45.72) (end 25.4 45.72) (width 1) (layer "B.Cu") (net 5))
 (segment (start 38.432 27.432) (end 39.37 28.37) (width 1) (layer "B.Cu") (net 5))
 (segment (start 30.5308 29.26) (end 28.0408 29.26) (width 1) (layer "B.Cu") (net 5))
 (segment (start 34.8488 27.432) (end 38.432 27.432) (width 1) (layer "B.Cu") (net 5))
 (segment (start 34.3908 29.21) (end 34.3908 31.7) (width 1) (layer "B.Cu") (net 5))
 (segment (start 27.94 44.45) (end 26.67 45.72) (width 1) (layer "B.Cu") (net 5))
 (segment (start 27.9908 43.865) (end 27.9908 41.275) (width 1) (layer "B.Cu") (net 5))
 (segment (start 34.3908 27.99) (end 34.3408 27.94) (width 1) (layer "B.Cu") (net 5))
 (segment (start 28.0408 29.26) (end 27.9908 29.21) (width 1) (layer "B.Cu") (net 5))
 (segment (start 30.5308 29.26) (end 34.3408 29.26) (width 1) (layer "B.Cu") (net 5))
 (segment (start 34.3408 27.94) (end 34.8488 27.432) (width 1) (layer "B.Cu") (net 5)))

